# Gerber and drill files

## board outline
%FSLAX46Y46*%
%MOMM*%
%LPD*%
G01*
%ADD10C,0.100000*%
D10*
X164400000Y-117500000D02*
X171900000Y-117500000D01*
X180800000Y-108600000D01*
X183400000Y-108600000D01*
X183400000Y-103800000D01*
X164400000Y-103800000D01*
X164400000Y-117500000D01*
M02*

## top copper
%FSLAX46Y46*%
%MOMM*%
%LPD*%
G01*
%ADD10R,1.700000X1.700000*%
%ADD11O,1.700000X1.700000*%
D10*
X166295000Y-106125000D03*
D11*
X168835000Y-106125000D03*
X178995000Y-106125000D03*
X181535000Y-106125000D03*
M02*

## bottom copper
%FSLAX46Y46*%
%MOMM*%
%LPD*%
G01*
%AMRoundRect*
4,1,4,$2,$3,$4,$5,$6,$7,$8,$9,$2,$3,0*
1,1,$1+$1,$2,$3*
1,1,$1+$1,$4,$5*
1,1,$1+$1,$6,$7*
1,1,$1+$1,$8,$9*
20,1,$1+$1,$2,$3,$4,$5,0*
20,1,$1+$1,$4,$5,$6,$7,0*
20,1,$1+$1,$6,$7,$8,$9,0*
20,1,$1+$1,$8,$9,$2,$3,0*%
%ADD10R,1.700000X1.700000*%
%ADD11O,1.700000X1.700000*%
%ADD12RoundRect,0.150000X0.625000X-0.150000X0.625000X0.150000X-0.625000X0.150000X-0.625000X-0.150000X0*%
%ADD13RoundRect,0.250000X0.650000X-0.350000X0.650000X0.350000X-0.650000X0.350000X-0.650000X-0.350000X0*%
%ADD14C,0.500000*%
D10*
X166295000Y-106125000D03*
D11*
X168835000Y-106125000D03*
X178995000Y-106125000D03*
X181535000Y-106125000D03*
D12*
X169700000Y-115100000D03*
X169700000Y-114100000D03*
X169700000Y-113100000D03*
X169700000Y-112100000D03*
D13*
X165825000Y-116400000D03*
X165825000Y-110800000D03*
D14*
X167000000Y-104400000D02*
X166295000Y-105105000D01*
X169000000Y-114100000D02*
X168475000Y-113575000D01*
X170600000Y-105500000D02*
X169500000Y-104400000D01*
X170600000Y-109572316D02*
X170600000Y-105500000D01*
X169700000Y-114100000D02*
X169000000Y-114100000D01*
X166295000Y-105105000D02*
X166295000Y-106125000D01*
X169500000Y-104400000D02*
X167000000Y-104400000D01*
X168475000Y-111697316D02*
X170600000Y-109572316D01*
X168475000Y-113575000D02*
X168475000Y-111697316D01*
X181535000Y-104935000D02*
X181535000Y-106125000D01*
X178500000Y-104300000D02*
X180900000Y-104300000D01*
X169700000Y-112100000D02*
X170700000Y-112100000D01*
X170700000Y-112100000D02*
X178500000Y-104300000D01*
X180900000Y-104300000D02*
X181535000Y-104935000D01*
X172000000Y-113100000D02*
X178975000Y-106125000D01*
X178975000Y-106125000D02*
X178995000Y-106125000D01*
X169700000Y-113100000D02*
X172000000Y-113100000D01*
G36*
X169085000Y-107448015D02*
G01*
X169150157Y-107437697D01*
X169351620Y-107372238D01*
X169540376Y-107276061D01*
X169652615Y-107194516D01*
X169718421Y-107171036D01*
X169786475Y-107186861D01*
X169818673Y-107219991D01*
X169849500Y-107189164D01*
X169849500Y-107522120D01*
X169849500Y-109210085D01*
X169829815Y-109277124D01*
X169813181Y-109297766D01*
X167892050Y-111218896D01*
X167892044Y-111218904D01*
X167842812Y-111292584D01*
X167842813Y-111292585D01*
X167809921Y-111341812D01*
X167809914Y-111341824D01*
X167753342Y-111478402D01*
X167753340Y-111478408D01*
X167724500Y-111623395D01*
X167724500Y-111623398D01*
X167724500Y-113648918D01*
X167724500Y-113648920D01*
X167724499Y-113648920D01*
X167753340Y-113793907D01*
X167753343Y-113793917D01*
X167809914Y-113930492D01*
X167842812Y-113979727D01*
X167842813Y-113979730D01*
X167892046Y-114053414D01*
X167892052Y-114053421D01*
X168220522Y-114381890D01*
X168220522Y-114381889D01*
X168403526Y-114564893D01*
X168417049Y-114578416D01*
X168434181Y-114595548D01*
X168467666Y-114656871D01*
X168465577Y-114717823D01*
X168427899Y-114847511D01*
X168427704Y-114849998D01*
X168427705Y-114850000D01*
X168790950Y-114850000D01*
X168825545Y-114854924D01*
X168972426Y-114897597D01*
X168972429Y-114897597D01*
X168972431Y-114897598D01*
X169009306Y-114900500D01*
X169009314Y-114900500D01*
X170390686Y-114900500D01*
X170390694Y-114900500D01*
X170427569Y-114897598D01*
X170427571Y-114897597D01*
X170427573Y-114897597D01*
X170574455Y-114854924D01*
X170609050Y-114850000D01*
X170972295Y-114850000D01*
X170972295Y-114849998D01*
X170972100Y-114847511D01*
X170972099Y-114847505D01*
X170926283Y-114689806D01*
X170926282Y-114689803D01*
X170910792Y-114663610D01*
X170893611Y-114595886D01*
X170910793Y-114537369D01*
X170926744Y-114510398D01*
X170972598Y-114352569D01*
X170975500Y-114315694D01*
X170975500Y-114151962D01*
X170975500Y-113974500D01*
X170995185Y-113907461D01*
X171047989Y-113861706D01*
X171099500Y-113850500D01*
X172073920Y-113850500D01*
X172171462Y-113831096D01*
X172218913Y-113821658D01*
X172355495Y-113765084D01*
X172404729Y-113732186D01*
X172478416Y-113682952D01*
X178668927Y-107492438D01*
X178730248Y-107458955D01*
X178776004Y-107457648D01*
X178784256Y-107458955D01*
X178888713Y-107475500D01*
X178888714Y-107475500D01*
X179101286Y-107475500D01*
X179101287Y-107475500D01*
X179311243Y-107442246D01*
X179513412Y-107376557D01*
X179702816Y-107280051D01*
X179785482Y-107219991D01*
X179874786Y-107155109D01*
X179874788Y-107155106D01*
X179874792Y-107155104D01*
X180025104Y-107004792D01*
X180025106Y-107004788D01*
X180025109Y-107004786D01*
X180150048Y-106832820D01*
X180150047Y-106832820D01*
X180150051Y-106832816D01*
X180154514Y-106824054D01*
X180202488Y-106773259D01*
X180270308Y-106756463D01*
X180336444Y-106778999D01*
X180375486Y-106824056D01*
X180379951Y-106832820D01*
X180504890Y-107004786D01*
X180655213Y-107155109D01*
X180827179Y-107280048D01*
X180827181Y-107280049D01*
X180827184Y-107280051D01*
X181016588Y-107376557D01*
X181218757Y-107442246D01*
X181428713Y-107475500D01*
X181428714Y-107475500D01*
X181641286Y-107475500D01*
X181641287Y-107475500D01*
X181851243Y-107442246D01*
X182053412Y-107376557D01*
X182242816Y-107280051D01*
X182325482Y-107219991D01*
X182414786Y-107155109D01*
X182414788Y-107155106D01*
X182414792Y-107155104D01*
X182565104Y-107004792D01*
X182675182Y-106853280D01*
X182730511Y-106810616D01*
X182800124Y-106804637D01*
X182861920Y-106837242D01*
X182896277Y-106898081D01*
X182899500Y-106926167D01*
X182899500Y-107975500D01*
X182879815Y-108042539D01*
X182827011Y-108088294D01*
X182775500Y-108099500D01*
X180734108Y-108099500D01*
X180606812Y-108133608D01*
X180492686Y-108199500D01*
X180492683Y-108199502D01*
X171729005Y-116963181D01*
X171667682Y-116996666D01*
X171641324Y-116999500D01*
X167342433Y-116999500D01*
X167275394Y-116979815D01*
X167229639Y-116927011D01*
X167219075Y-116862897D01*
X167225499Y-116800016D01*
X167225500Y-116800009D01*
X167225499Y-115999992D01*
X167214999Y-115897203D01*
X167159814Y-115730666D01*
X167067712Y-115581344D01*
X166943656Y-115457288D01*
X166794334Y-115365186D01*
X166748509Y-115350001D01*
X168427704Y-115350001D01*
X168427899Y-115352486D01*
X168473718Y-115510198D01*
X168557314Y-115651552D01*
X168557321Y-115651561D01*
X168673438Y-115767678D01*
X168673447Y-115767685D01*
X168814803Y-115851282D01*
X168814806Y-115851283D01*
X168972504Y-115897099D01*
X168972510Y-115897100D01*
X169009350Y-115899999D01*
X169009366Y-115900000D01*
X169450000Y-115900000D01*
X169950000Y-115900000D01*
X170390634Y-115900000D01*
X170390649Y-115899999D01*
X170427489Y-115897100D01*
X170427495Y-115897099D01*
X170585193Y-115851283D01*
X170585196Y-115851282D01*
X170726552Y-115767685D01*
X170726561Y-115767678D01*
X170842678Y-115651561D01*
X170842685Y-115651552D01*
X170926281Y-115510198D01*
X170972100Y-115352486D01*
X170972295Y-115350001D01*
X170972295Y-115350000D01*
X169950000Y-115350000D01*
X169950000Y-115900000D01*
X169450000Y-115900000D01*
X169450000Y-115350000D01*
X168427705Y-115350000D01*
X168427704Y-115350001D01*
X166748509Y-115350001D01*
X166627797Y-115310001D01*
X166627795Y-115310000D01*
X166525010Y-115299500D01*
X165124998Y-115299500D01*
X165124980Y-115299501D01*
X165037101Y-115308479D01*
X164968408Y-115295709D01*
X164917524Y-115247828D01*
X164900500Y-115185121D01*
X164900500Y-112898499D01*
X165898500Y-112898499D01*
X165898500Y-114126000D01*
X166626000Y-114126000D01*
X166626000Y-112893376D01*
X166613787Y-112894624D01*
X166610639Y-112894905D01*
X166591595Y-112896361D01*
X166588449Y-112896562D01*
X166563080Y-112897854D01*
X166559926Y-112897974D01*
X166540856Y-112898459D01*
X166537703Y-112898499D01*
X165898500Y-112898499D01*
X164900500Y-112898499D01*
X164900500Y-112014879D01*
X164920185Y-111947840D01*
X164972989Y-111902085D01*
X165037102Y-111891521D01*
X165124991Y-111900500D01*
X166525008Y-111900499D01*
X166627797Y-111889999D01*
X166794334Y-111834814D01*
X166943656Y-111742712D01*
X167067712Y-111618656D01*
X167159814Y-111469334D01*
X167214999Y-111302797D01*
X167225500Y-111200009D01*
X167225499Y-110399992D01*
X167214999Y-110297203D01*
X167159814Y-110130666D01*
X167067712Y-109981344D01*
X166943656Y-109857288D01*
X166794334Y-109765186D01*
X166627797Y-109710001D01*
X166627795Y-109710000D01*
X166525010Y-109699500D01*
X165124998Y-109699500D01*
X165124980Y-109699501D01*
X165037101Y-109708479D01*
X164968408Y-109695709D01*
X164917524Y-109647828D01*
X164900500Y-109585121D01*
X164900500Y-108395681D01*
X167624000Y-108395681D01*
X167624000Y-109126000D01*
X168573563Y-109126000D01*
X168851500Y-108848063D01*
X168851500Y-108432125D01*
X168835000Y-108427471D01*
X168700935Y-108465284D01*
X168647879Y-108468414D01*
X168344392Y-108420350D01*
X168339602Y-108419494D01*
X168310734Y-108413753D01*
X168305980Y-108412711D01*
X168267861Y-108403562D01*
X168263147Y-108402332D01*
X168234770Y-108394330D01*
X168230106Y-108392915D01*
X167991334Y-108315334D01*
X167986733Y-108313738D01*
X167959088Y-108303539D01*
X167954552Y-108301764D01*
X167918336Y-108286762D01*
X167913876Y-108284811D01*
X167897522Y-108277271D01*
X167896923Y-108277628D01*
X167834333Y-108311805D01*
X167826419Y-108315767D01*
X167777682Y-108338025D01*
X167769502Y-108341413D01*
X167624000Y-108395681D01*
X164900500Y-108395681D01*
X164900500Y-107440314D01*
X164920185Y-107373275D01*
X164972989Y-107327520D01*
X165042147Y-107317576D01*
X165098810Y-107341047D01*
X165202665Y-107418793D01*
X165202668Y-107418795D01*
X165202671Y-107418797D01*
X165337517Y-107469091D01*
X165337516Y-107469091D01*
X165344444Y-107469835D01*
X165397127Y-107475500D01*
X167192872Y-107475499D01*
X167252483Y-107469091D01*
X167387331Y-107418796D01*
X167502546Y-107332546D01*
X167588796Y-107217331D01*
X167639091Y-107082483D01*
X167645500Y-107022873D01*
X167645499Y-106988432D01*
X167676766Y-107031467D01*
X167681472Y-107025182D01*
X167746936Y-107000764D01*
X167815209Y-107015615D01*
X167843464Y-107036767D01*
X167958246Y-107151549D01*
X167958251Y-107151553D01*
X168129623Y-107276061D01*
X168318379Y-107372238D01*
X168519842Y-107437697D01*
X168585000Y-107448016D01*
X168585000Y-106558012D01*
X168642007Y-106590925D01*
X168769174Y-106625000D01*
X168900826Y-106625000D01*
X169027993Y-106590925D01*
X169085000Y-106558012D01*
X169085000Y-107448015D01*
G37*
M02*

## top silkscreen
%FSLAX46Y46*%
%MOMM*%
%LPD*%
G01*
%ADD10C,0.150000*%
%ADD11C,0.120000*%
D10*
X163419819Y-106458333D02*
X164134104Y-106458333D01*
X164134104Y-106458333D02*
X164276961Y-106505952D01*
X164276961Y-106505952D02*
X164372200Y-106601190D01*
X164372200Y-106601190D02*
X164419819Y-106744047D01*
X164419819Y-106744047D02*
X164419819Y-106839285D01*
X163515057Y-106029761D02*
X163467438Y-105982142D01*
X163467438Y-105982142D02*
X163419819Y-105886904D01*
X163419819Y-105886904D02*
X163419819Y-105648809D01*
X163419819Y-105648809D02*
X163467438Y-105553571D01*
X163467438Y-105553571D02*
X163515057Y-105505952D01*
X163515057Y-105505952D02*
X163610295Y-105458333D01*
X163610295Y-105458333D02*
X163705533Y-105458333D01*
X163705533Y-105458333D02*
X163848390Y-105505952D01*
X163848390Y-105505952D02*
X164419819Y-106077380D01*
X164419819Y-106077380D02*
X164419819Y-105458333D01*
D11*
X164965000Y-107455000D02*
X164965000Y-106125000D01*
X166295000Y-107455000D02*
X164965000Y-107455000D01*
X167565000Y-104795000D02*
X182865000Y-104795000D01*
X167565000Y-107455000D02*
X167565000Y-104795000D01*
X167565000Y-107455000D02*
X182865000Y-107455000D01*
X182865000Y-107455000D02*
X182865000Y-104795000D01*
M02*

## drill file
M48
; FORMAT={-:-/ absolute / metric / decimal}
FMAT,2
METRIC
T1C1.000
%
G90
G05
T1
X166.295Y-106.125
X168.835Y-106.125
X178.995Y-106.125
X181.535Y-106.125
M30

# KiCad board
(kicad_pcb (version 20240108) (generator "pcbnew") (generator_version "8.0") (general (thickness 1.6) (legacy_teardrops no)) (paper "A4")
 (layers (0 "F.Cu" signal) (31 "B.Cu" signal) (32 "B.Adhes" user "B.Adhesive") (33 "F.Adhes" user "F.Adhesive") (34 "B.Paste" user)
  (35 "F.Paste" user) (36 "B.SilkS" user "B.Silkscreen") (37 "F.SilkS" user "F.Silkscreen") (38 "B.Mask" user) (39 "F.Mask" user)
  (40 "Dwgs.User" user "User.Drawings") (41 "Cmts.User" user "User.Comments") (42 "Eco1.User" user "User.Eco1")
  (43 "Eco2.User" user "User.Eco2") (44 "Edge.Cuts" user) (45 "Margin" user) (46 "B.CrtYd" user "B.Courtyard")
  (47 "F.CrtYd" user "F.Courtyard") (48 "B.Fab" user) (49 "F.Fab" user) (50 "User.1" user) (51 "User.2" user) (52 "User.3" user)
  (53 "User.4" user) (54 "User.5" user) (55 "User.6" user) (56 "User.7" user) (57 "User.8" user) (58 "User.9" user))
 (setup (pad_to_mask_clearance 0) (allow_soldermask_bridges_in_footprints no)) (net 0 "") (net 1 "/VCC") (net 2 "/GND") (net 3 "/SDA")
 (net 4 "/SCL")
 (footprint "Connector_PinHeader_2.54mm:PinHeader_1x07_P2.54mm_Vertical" (layer "F.Cu") (at 166.295 106.125 90)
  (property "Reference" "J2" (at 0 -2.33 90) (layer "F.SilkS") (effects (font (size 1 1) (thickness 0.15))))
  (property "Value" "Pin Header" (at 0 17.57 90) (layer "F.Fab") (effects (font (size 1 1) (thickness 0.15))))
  (fp_line (start -1.33 -1.33) (end 0 -1.33) (stroke (width 0.12) (type solid)) (layer "F.SilkS"))
  (fp_line (start -1.33 0) (end -1.33 -1.33) (stroke (width 0.12) (type solid)) (layer "F.SilkS"))
  (fp_line (start 1.33 1.27) (end 1.33 16.57) (stroke (width 0.12) (type solid)) (layer "F.SilkS"))
  (fp_line (start -1.33 1.27) (end 1.33 1.27) (stroke (width 0.12) (type solid)) (layer "F.SilkS"))
  (fp_line (start -1.33 1.27) (end -1.33 16.57) (stroke (width 0.12) (type solid)) (layer "F.SilkS"))
  (fp_line (start -1.33 16.57) (end 1.33 16.57) (stroke (width 0.12) (type solid)) (layer "F.SilkS"))
  (pad "1" thru_hole rect (at 0 0 90) (size 1.7 1.7) (drill 1) (layers "*.Cu" "*.Mask") (remove_unused_layers no) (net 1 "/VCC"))
  (pad "2" thru_hole oval (at 0 2.54 90) (size 1.7 1.7) (drill 1) (layers "*.Cu" "*.Mask") (remove_unused_layers no) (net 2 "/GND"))
  (pad "6" thru_hole oval (at 0 12.7 90) (size 1.7 1.7) (drill 1) (layers "*.Cu" "*.Mask") (remove_unused_layers no) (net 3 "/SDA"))
  (pad "7" thru_hole oval (at 0 15.24 90) (size 1.7 1.7) (drill 1) (layers "*.Cu" "*.Mask") (remove_unused_layers no) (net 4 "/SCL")))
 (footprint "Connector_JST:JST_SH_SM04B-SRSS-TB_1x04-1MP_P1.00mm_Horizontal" (layer "B.Cu") (at 167.7 113.6 90)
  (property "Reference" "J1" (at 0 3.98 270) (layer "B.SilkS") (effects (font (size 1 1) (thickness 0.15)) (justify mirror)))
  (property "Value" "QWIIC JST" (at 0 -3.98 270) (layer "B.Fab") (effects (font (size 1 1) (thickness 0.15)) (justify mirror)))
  (pad "1" smd roundrect (at -1.5 2 90) (size 0.6 1.55) (layers "B.Cu" "B.Paste" "B.Mask") (roundrect_rratio 0.25) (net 2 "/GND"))
  (pad "2" smd roundrect (at -0.5 2 90) (size 0.6 1.55) (layers "B.Cu" "B.Paste" "B.Mask") (roundrect_rratio 0.25) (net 1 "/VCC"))
  (pad "3" smd roundrect (at 0.5 2 90) (size 0.6 1.55) (layers "B.Cu" "B.Paste" "B.Mask") (roundrect_rratio 0.25) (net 3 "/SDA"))
  (pad "4" smd roundrect (at 1.5 2 90) (size 0.6 1.55) (layers "B.Cu" "B.Paste" "B.Mask") (roundrect_rratio 0.25) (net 4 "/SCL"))
  (pad "MP" smd roundrect (at -2.8 -1.875 90) (size 1.2 1.8) (layers "B.Cu" "B.Paste" "B.Mask") (roundrect_rratio 0.208333))
  (pad "MP" smd roundrect (at 2.8 -1.875 90) (size 1.2 1.8) (layers "B.Cu" "B.Paste" "B.Mask") (roundrect_rratio 0.208333)))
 (gr_poly
  (pts (xy 164.4 117.5) (xy 171.9 117.5) (xy 180.8 108.6) (xy 183.4 108.6) (xy 183.4 103.8) (xy 164.4 103.8))
  (stroke (width 0.1) (type solid)) (fill none) (layer "Edge.Cuts"))
 (segment (start 167 104.4) (end 166.295 105.105) (width 0.5) (layer "B.Cu") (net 1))
 (segment (start 169 114.1) (end 168.475 113.575) (width 0.5) (layer "B.Cu") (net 1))
 (segment (start 170.6 105.5) (end 169.5 104.4) (width 0.5) (layer "B.Cu") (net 1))
 (segment (start 170.6 109.572316) (end 170.6 105.5) (width 0.5) (layer "B.Cu") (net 1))
 (segment (start 169.7 114.1) (end 169 114.1) (width 0.5) (layer "B.Cu") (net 1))
 (segment (start 166.295 105.105) (end 166.295 106.125) (width 0.5) (layer "B.Cu") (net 1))
 (segment (start 169.5 104.4) (end 167 104.4) (width 0.5) (layer "B.Cu") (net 1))
 (segment (start 168.475 111.697316) (end 170.6 109.572316) (width 0.5) (layer "B.Cu") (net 1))
 (segment (start 168.475 113.575) (end 168.475 111.697316) (width 0.5) (layer "B.Cu") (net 1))
 (segment (start 181.535 104.935) (end 181.535 106.125) (width 0.5) (layer "B.Cu") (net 4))
 (segment (start 178.5 104.3) (end 180.9 104.3) (width 0.5) (layer "B.Cu") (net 4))
 (segment (start 169.7 112.1) (end 170.7 112.1) (width 0.5) (layer "B.Cu") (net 4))
 (segment (start 170.7 112.1) (end 178.5 104.3) (width 0.5) (layer "B.Cu") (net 4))
 (segment (start 180.9 104.3) (end 181.535 104.935) (width 0.5) (layer "B.Cu") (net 4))
 (segment (start 172 113.1) (end 178.975 106.125) (width 0.5) (layer "B.Cu") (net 3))
 (segment (start 178.975 106.125) (end 178.995 106.125) (width 0.5) (layer "B.Cu") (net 3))
 (segment (start 169.7 113.1) (end 172 113.1) (width 0.5) (layer "B.Cu") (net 3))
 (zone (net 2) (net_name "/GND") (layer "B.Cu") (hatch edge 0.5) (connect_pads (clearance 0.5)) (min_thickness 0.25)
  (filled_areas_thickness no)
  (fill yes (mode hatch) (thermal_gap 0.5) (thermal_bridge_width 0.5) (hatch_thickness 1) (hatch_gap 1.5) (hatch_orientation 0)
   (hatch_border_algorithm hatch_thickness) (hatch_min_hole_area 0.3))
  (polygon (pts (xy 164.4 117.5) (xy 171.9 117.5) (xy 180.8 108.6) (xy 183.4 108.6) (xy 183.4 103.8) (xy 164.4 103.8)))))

